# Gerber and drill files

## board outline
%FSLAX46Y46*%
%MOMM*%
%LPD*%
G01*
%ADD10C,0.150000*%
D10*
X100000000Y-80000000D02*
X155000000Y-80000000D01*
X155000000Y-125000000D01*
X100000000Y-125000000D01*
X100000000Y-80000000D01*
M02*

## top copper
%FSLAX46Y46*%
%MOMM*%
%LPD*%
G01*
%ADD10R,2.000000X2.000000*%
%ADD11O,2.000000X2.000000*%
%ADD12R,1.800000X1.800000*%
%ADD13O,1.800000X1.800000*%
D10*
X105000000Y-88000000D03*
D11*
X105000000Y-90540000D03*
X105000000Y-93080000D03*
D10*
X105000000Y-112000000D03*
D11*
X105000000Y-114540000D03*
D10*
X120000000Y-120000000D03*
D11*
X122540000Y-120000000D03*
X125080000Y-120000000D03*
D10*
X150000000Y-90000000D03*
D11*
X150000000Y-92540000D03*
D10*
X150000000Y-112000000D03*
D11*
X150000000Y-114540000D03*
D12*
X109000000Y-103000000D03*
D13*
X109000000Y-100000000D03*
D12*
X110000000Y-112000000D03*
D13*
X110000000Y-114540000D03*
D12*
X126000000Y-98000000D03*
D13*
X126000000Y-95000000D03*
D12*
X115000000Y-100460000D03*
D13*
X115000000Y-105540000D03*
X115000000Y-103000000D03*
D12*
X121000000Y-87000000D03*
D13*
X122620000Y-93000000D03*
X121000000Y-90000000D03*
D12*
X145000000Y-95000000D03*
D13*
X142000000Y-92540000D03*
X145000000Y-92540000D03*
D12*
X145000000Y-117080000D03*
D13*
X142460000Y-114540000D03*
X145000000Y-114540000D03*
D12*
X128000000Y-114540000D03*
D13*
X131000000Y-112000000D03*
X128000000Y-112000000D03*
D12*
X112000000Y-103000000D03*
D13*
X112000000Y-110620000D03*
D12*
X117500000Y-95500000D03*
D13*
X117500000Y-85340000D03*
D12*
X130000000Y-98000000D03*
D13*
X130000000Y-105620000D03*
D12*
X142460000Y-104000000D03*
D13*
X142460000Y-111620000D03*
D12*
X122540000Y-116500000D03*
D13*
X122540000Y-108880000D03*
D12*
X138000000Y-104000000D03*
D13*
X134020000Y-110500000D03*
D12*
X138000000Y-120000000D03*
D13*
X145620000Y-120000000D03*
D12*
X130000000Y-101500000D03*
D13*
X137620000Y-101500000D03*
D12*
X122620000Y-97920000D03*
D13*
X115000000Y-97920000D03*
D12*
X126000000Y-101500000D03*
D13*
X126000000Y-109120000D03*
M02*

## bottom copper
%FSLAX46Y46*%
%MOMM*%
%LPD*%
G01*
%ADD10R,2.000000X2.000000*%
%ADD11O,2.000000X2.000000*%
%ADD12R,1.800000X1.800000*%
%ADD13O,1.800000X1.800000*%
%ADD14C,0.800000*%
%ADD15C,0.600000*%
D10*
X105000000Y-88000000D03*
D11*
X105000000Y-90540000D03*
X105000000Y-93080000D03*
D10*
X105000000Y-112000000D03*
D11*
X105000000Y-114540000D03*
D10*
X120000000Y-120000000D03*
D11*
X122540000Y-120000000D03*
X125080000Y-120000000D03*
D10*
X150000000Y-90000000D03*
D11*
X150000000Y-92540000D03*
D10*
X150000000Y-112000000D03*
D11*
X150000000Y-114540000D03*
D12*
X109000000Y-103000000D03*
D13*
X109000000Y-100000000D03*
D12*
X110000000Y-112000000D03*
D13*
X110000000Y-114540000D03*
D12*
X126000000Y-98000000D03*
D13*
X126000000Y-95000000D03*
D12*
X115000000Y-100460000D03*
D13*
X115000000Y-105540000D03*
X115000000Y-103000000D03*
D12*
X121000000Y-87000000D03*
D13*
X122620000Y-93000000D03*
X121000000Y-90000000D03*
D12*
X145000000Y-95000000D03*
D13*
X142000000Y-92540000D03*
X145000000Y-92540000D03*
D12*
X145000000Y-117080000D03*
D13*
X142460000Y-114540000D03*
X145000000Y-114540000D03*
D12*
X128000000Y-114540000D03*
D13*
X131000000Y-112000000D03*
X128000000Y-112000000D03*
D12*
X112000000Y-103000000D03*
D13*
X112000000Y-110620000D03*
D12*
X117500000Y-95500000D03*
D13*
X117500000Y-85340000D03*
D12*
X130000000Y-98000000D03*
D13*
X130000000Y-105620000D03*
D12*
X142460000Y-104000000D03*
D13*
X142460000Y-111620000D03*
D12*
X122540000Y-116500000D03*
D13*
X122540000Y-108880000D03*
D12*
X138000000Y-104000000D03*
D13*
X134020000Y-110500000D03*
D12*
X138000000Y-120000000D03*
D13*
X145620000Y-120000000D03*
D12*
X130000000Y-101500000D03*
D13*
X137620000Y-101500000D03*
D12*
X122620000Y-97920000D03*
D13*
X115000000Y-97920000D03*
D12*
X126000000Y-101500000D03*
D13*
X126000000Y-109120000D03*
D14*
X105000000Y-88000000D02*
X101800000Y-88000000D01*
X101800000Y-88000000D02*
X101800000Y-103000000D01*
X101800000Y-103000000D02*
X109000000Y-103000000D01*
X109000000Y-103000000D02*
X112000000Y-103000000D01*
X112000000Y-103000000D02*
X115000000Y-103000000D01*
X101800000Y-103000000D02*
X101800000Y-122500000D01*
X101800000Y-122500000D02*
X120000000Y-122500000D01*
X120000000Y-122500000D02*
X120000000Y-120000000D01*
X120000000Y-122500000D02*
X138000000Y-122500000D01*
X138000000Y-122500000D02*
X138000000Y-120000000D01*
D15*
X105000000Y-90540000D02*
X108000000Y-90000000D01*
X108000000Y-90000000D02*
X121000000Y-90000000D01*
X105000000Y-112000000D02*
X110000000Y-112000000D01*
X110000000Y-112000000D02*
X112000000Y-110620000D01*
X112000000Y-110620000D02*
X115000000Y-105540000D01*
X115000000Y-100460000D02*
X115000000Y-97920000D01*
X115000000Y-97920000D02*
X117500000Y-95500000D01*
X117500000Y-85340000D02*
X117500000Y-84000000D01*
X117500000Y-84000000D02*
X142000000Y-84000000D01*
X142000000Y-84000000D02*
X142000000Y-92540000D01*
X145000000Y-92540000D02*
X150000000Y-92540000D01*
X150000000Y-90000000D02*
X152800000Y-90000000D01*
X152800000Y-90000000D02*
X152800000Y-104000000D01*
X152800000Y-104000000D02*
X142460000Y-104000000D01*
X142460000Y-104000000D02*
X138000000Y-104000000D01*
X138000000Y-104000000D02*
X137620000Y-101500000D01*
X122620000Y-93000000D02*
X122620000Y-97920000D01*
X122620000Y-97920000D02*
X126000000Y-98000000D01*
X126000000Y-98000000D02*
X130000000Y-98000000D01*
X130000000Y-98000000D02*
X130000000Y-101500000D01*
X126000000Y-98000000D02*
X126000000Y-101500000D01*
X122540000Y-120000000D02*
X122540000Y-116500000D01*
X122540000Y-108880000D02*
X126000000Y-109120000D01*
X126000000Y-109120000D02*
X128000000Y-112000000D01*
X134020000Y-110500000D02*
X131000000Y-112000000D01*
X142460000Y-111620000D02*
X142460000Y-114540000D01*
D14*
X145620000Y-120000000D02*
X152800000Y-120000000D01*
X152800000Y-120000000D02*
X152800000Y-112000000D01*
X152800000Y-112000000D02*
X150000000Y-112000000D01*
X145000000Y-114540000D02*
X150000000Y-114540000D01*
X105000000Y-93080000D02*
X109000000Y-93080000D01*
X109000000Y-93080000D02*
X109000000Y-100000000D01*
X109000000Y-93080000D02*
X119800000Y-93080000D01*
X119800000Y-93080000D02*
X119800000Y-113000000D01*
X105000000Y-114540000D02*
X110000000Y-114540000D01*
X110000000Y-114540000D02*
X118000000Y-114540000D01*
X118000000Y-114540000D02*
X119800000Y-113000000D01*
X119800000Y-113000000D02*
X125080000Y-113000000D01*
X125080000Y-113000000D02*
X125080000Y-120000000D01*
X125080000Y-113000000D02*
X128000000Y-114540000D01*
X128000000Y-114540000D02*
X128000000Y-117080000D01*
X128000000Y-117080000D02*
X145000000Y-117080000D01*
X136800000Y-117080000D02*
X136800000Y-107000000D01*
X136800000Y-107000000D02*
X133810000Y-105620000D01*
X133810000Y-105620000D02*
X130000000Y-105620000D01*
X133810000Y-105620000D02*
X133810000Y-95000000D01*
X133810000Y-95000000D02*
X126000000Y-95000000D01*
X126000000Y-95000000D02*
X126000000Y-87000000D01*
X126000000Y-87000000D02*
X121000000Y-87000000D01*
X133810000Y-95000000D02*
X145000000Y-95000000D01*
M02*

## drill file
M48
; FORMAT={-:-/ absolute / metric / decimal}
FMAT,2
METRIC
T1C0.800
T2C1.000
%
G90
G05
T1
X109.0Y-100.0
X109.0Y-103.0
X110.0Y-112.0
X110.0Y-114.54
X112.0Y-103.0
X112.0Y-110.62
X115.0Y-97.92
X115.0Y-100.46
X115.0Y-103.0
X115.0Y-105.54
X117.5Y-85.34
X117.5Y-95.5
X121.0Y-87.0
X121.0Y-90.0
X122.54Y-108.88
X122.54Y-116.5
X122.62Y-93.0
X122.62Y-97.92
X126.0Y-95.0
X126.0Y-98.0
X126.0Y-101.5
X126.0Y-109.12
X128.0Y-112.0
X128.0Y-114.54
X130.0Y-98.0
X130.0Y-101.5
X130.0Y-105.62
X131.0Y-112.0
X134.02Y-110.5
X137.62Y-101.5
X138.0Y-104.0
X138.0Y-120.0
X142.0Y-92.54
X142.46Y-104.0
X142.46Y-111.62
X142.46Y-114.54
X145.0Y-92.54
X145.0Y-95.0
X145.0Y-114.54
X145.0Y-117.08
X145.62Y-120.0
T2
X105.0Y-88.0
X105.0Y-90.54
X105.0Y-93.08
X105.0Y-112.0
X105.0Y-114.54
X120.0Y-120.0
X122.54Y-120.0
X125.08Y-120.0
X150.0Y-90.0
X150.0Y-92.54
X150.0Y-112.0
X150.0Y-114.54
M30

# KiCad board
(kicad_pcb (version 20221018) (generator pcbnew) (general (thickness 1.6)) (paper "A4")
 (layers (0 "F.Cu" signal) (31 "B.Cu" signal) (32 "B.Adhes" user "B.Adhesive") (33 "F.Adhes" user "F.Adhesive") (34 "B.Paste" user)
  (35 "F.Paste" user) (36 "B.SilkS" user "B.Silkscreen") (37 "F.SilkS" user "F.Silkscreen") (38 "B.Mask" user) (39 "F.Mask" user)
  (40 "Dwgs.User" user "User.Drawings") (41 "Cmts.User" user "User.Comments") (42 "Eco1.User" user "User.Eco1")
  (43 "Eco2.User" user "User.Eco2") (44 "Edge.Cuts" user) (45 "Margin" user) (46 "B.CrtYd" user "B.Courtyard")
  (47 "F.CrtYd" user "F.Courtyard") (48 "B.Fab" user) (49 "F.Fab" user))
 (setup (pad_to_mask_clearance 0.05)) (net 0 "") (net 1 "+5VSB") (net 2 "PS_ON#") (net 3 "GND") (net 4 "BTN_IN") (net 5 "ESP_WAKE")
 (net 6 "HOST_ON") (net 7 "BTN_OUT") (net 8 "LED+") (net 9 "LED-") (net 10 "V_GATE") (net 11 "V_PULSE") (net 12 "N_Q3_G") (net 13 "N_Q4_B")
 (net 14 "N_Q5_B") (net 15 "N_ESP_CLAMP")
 (gr_rect (start 100 80) (end 155 125) (layer "Edge.Cuts") (width 0.15) (fill none))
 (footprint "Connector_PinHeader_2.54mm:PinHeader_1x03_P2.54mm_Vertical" (layer "F.Cu") (at 105.00 88.00)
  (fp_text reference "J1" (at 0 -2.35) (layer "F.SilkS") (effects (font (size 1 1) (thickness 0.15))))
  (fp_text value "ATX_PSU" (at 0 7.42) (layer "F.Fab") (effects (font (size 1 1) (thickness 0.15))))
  (pad "1" thru_hole rect (at 0.00 0.00) (size 2.00 2.00) (drill 1.00) (layers "B.Cu" "B.Mask") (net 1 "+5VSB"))
  (pad "2" thru_hole oval (at 0.00 2.54) (size 2.00 2.00) (drill 1.00) (layers "B.Cu" "B.Mask") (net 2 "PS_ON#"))
  (pad "3" thru_hole oval (at 0.00 5.08) (size 2.00 2.00) (drill 1.00) (layers "B.Cu" "B.Mask") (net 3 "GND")))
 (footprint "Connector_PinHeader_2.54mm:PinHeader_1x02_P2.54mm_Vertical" (layer "F.Cu") (at 105.00 112.00)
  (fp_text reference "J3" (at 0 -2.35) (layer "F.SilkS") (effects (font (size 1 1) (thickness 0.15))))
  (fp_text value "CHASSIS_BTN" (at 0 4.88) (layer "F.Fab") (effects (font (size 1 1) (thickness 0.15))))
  (pad "1" thru_hole rect (at 0.00 0.00) (size 2.00 2.00) (drill 1.00) (layers "B.Cu" "B.Mask") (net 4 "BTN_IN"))
  (pad "2" thru_hole oval (at 0.00 2.54) (size 2.00 2.00) (drill 1.00) (layers "B.Cu" "B.Mask") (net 3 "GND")))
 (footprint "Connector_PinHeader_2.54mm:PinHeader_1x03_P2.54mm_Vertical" (layer "F.Cu") (at 120.00 120.00)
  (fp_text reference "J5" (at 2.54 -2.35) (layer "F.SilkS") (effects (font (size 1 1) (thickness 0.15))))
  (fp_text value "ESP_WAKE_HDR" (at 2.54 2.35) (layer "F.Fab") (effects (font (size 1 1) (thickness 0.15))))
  (pad "1" thru_hole rect (at 0.00 0.00) (size 2.00 2.00) (drill 1.00) (layers "B.Cu" "B.Mask") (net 1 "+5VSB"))
  (pad "2" thru_hole oval (at 2.54 0.00) (size 2.00 2.00) (drill 1.00) (layers "B.Cu" "B.Mask") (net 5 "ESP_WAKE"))
  (pad "3" thru_hole oval (at 5.08 0.00) (size 2.00 2.00) (drill 1.00) (layers "B.Cu" "B.Mask") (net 3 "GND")))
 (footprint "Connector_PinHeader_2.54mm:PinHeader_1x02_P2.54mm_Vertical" (layer "F.Cu") (at 150.00 90.00)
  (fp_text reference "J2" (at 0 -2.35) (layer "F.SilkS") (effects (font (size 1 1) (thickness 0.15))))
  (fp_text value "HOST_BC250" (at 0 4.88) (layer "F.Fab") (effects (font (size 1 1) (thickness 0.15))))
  (pad "1" thru_hole rect (at 0.00 0.00) (size 2.00 2.00) (drill 1.00) (layers "B.Cu" "B.Mask") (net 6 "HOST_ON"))
  (pad "2" thru_hole oval (at 0.00 2.54) (size 2.00 2.00) (drill 1.00) (layers "B.Cu" "B.Mask") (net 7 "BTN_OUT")))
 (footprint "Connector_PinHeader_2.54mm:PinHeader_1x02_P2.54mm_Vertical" (layer "F.Cu") (at 150.00 112.00)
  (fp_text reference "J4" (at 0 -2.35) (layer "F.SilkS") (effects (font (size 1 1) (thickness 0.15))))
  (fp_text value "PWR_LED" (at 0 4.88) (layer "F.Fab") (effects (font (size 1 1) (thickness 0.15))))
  (pad "1" thru_hole rect (at 0.00 0.00) (size 2.00 2.00) (drill 1.00) (layers "B.Cu" "B.Mask") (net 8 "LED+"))
  (pad "2" thru_hole oval (at 0.00 2.54) (size 2.00 2.00) (drill 1.00) (layers "B.Cu" "B.Mask") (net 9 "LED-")))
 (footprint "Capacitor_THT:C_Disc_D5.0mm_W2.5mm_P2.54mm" (layer "F.Cu") (at 109.00 103.00)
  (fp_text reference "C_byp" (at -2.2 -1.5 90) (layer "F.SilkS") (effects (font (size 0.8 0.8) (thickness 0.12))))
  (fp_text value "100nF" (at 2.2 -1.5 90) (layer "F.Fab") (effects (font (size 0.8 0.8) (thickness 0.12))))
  (pad "1" thru_hole rect (at 0.00 0.00) (size 1.80 1.80) (drill 0.80) (layers "B.Cu" "B.Mask") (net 1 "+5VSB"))
  (pad "2" thru_hole oval (at 0.00 -3.00) (size 1.80 1.80) (drill 0.80) (layers "B.Cu" "B.Mask") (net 3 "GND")))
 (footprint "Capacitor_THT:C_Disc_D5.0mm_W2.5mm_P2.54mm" (layer "F.Cu") (at 110.00 112.00)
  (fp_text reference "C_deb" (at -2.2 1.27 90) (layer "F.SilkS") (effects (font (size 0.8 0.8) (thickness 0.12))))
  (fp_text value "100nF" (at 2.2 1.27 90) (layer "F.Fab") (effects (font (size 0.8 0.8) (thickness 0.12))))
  (pad "1" thru_hole rect (at 0.00 0.00) (size 1.80 1.80) (drill 0.80) (layers "B.Cu" "B.Mask") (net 4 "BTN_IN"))
  (pad "2" thru_hole oval (at 0.00 2.54) (size 1.80 1.80) (drill 0.80) (layers "B.Cu" "B.Mask") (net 3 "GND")))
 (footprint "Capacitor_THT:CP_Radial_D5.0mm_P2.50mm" (layer "F.Cu") (at 126.00 98.00)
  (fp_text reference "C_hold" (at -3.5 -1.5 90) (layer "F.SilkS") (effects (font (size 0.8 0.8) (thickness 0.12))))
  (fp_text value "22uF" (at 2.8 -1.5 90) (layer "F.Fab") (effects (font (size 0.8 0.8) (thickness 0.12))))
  (pad "1" thru_hole rect (at 0.00 0.00) (size 1.80 1.80) (drill 0.80) (layers "B.Cu" "B.Mask") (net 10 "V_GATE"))
  (pad "2" thru_hole oval (at 0.00 -3.00) (size 1.80 1.80) (drill 0.80) (layers "B.Cu" "B.Mask") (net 3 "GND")))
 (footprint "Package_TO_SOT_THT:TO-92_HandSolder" (layer "F.Cu") (at 115.00 103.00)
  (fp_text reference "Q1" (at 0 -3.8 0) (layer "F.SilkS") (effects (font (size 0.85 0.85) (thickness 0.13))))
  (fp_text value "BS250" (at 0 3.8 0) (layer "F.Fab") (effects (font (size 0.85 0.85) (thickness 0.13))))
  (pad "1" thru_hole rect (at 0.00 -2.54) (size 1.80 1.80) (drill 0.80) (layers "B.Cu" "B.Mask") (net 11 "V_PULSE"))
  (pad "2" thru_hole oval (at 0.00 2.54) (size 1.80 1.80) (drill 0.80) (layers "B.Cu" "B.Mask") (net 4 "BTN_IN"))
  (pad "3" thru_hole oval (at 0.00 0.00) (size 1.80 1.80) (drill 0.80) (layers "B.Cu" "B.Mask") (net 1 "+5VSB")))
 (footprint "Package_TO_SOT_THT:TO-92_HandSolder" (layer "F.Cu") (at 121.00 90.00)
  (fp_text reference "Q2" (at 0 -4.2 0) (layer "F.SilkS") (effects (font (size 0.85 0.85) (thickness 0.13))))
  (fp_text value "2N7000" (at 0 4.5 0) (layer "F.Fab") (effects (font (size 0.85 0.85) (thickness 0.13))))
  (pad "1" thru_hole rect (at 0.00 -3.00) (size 1.80 1.80) (drill 0.80) (layers "B.Cu" "B.Mask") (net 3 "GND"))
  (pad "2" thru_hole oval (at 1.62 3.00) (size 1.80 1.80) (drill 0.80) (layers "B.Cu" "B.Mask") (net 10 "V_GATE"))
  (pad "3" thru_hole oval (at 0.00 0.00) (size 1.80 1.80) (drill 0.80) (layers "B.Cu" "B.Mask") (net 2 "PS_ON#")))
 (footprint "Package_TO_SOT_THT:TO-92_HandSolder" (layer "F.Cu") (at 145.00 92.54)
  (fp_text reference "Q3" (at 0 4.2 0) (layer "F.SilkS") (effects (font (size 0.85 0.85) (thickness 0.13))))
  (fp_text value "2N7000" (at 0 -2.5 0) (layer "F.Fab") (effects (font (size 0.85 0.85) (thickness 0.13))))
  (pad "1" thru_hole rect (at 0.00 2.46) (size 1.80 1.80) (drill 0.80) (layers "B.Cu" "B.Mask") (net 3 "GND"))
  (pad "2" thru_hole oval (at -3.00 0.00) (size 1.80 1.80) (drill 0.80) (layers "B.Cu" "B.Mask") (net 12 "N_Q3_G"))
  (pad "3" thru_hole oval (at 0.00 0.00) (size 1.80 1.80) (drill 0.80) (layers "B.Cu" "B.Mask") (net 7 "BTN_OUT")))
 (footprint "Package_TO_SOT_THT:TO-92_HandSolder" (layer "F.Cu") (at 145.00 114.54)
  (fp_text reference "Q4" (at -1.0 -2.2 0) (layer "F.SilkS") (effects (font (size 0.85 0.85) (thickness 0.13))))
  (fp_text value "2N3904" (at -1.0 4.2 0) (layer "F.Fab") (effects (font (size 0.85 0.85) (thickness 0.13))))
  (pad "1" thru_hole rect (at 0.00 2.54) (size 1.80 1.80) (drill 0.80) (layers "B.Cu" "B.Mask") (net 3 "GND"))
  (pad "2" thru_hole oval (at -2.54 0.00) (size 1.80 1.80) (drill 0.80) (layers "B.Cu" "B.Mask") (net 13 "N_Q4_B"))
  (pad "3" thru_hole oval (at 0.00 0.00) (size 1.80 1.80) (drill 0.80) (layers "B.Cu" "B.Mask") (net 9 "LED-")))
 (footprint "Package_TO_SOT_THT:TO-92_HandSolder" (layer "F.Cu") (at 128.00 112.00)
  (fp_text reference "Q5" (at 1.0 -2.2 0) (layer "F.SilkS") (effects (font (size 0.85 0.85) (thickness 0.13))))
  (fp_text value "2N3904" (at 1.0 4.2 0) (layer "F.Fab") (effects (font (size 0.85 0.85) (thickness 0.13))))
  (pad "1" thru_hole rect (at 0.00 2.54) (size 1.80 1.80) (drill 0.80) (layers "B.Cu" "B.Mask") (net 3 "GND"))
  (pad "2" thru_hole oval (at 3.00 0.00) (size 1.80 1.80) (drill 0.80) (layers "B.Cu" "B.Mask") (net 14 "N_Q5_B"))
  (pad "3" thru_hole oval (at 0.00 0.00) (size 1.80 1.80) (drill 0.80) (layers "B.Cu" "B.Mask") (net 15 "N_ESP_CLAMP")))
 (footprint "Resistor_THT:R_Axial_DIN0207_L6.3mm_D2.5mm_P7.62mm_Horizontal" (layer "F.Cu") (at 112.00 103.00)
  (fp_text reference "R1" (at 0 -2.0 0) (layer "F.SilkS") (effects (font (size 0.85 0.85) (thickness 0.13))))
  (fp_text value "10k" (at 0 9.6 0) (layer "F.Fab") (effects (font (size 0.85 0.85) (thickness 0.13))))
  (pad "1" thru_hole rect (at 0.00 0.00) (size 1.80 1.80) (drill 0.80) (layers "B.Cu" "B.Mask") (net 1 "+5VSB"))
  (pad "2" thru_hole oval (at 0.00 7.62) (size 1.80 1.80) (drill 0.80) (layers "B.Cu" "B.Mask") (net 4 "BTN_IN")))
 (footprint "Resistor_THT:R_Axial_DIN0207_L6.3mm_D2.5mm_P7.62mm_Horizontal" (layer "F.Cu") (at 117.50 95.50)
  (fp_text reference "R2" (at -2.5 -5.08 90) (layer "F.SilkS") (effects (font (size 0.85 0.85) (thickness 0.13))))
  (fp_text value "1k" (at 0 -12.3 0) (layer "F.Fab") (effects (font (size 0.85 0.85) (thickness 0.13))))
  (pad "1" thru_hole rect (at 0.00 0.00) (size 1.80 1.80) (drill 0.80) (layers "B.Cu" "B.Mask") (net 11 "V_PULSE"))
  (pad "2" thru_hole oval (at 0.00 -10.16) (size 1.80 1.80) (drill 0.80) (layers "B.Cu" "B.Mask") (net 12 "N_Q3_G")))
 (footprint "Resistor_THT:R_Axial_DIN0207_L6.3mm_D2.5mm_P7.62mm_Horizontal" (layer "F.Cu") (at 130.00 98.00)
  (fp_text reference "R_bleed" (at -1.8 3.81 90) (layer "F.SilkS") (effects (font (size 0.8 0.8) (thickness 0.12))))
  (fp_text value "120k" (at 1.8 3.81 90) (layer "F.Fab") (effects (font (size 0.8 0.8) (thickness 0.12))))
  (pad "1" thru_hole rect (at 0.00 0.00) (size 1.80 1.80) (drill 0.80) (layers "B.Cu" "B.Mask") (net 10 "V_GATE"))
  (pad "2" thru_hole oval (at 0.00 7.62) (size 1.80 1.80) (drill 0.80) (layers "B.Cu" "B.Mask") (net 3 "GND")))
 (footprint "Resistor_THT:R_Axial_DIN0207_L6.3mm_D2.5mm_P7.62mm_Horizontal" (layer "F.Cu") (at 142.46 104.00)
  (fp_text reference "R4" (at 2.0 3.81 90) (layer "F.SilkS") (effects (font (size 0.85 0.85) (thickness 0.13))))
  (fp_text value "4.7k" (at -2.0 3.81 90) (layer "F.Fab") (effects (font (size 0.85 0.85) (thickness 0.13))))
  (pad "1" thru_hole rect (at 0.00 0.00) (size 1.80 1.80) (drill 0.80) (layers "B.Cu" "B.Mask") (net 6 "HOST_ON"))
  (pad "2" thru_hole oval (at 0.00 7.62) (size 1.80 1.80) (drill 0.80) (layers "B.Cu" "B.Mask") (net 13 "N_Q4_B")))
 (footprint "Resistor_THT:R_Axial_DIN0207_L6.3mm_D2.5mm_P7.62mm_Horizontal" (layer "F.Cu") (at 122.54 116.50)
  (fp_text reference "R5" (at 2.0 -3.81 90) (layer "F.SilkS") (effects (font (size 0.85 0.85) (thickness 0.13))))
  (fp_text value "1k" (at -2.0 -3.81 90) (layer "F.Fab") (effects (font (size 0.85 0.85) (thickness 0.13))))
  (pad "1" thru_hole rect (at 0.00 0.00) (size 1.80 1.80) (drill 0.80) (layers "B.Cu" "B.Mask") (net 5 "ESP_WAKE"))
  (pad "2" thru_hole oval (at 0.00 -7.62) (size 1.80 1.80) (drill 0.80) (layers "B.Cu" "B.Mask") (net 15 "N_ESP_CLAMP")))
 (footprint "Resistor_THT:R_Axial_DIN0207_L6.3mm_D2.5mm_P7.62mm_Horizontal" (layer "F.Cu") (at 138.00 104.00)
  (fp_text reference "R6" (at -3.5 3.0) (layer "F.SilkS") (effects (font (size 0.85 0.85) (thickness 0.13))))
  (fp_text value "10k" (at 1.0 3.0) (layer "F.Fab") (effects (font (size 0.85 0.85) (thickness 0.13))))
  (pad "1" thru_hole rect (at 0.00 0.00) (size 1.80 1.80) (drill 0.80) (layers "B.Cu" "B.Mask") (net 6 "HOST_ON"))
  (pad "2" thru_hole oval (at -3.98 6.50) (size 1.80 1.80) (drill 0.80) (layers "B.Cu" "B.Mask") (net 14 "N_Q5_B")))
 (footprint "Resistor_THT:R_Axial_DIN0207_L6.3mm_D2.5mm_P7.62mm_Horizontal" (layer "F.Cu") (at 138.00 120.00)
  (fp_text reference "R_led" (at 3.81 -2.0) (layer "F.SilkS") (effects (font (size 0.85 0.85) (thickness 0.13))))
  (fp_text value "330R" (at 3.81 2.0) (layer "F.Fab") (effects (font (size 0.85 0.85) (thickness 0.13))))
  (pad "1" thru_hole rect (at 0.00 0.00) (size 1.80 1.80) (drill 0.80) (layers "B.Cu" "B.Mask") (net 1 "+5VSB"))
  (pad "2" thru_hole oval (at 7.62 0.00) (size 1.80 1.80) (drill 0.80) (layers "B.Cu" "B.Mask") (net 8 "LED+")))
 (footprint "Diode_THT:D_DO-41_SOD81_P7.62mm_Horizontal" (layer "F.Cu") (at 130.00 101.50)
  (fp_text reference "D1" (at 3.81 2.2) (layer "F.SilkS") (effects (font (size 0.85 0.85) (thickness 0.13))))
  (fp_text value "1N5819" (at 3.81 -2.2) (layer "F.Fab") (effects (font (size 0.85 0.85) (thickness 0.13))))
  (pad "1" thru_hole rect (at 0.00 0.00) (size 1.80 1.80) (drill 0.80) (layers "B.Cu" "B.Mask") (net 10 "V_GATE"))
  (pad "2" thru_hole oval (at 7.62 0.00) (size 1.80 1.80) (drill 0.80) (layers "B.Cu" "B.Mask") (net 6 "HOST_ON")))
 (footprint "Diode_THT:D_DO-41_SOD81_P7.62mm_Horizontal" (layer "F.Cu") (at 122.62 97.92)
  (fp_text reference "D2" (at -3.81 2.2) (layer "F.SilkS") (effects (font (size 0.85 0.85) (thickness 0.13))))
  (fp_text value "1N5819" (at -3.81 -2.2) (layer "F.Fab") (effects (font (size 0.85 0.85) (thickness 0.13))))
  (pad "1" thru_hole rect (at 0.00 0.00) (size 1.80 1.80) (drill 0.80) (layers "B.Cu" "B.Mask") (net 10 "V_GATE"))
  (pad "2" thru_hole oval (at -7.62 0.00) (size 1.80 1.80) (drill 0.80) (layers "B.Cu" "B.Mask") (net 11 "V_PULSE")))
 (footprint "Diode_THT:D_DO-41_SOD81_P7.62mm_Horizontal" (layer "F.Cu") (at 126.00 101.50)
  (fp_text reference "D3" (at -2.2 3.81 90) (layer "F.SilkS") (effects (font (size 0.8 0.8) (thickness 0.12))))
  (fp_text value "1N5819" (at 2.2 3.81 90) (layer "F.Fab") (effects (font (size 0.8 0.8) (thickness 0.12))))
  (pad "1" thru_hole rect (at 0.00 0.00) (size 1.80 1.80) (drill 0.80) (layers "B.Cu" "B.Mask") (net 10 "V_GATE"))
  (pad "2" thru_hole oval (at 0.00 7.62) (size 1.80 1.80) (drill 0.80) (layers "B.Cu" "B.Mask") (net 15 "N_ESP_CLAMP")))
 (segment (start 105.00 88.00) (end 101.80 88.00) (width 0.80) (layer "B.Cu") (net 1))
 (segment (start 101.80 88.00) (end 101.80 103.00) (width 0.80) (layer "B.Cu") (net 1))
 (segment (start 101.80 103.00) (end 109.00 103.00) (width 0.80) (layer "B.Cu") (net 1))
 (segment (start 109.00 103.00) (end 112.00 103.00) (width 0.80) (layer "B.Cu") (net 1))
 (segment (start 112.00 103.00) (end 115.00 103.00) (width 0.80) (layer "B.Cu") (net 1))
 (segment (start 101.80 103.00) (end 101.80 122.50) (width 0.80) (layer "B.Cu") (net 1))
 (segment (start 101.80 122.50) (end 120.00 122.50) (width 0.80) (layer "B.Cu") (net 1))
 (segment (start 120.00 122.50) (end 120.00 120.00) (width 0.80) (layer "B.Cu") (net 1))
 (segment (start 120.00 122.50) (end 138.00 122.50) (width 0.80) (layer "B.Cu") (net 1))
 (segment (start 138.00 122.50) (end 138.00 120.00) (width 0.80) (layer "B.Cu") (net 1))
 (segment (start 105.00 90.54) (end 108.00 90.00) (width 0.60) (layer "B.Cu") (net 2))
 (segment (start 108.00 90.00) (end 121.00 90.00) (width 0.60) (layer "B.Cu") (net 2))
 (segment (start 105.00 112.00) (end 110.00 112.00) (width 0.60) (layer "B.Cu") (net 4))
 (segment (start 110.00 112.00) (end 112.00 110.62) (width 0.60) (layer "B.Cu") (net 4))
 (segment (start 112.00 110.62) (end 115.00 105.54) (width 0.60) (layer "B.Cu") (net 4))
 (segment (start 115.00 100.46) (end 115.00 97.92) (width 0.60) (layer "B.Cu") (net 11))
 (segment (start 115.00 97.92) (end 117.50 95.50) (width 0.60) (layer "B.Cu") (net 11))
 (segment (start 117.50 85.34) (end 117.50 84.00) (width 0.60) (layer "B.Cu") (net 12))
 (segment (start 117.50 84.00) (end 142.00 84.00) (width 0.60) (layer "B.Cu") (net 12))
 (segment (start 142.00 84.00) (end 142.00 92.54) (width 0.60) (layer "B.Cu") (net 12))
 (segment (start 145.00 92.54) (end 150.00 92.54) (width 0.60) (layer "B.Cu") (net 7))
 (segment (start 150.00 90.00) (end 152.80 90.00) (width 0.60) (layer "B.Cu") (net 6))
 (segment (start 152.80 90.00) (end 152.80 104.00) (width 0.60) (layer "B.Cu") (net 6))
 (segment (start 152.80 104.00) (end 142.46 104.00) (width 0.60) (layer "B.Cu") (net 6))
 (segment (start 142.46 104.00) (end 138.00 104.00) (width 0.60) (layer "B.Cu") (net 6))
 (segment (start 138.00 104.00) (end 137.62 101.50) (width 0.60) (layer "B.Cu") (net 6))
 (segment (start 122.62 93.00) (end 122.62 97.92) (width 0.60) (layer "B.Cu") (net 10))
 (segment (start 122.62 97.92) (end 126.00 98.00) (width 0.60) (layer "B.Cu") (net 10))
 (segment (start 126.00 98.00) (end 130.00 98.00) (width 0.60) (layer "B.Cu") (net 10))
 (segment (start 130.00 98.00) (end 130.00 101.50) (width 0.60) (layer "B.Cu") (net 10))
 (segment (start 126.00 98.00) (end 126.00 101.50) (width 0.60) (layer "B.Cu") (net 10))
 (segment (start 122.54 120.00) (end 122.54 116.50) (width 0.60) (layer "B.Cu") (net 5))
 (segment (start 122.54 108.88) (end 126.00 109.12) (width 0.60) (layer "B.Cu") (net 15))
 (segment (start 126.00 109.12) (end 128.00 112.00) (width 0.60) (layer "B.Cu") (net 15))
 (segment (start 134.02 110.50) (end 131.00 112.00) (width 0.60) (layer "B.Cu") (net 14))
 (segment (start 142.46 111.62) (end 142.46 114.54) (width 0.60) (layer "B.Cu") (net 13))
 (segment (start 145.62 120.00) (end 152.80 120.00) (width 0.80) (layer "B.Cu") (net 8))
 (segment (start 152.80 120.00) (end 152.80 112.00) (width 0.80) (layer "B.Cu") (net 8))
 (segment (start 152.80 112.00) (end 150.00 112.00) (width 0.80) (layer "B.Cu") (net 8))
 (segment (start 145.00 114.54) (end 150.00 114.54) (width 0.80) (layer "B.Cu") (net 9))
 (segment (start 105.00 93.08) (end 109.00 93.08) (width 0.80) (layer "B.Cu") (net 3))
 (segment (start 109.00 93.08) (end 109.00 100.00) (width 0.80) (layer "B.Cu") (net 3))
 (segment (start 109.00 93.08) (end 119.80 93.08) (width 0.80) (layer "B.Cu") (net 3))
 (segment (start 119.80 93.08) (end 119.80 113.00) (width 0.80) (layer "B.Cu") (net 3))
 (segment (start 105.00 114.54) (end 110.00 114.54) (width 0.80) (layer "B.Cu") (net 3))
 (segment (start 110.00 114.54) (end 118.00 114.54) (width 0.80) (layer "B.Cu") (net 3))
 (segment (start 118.00 114.54) (end 119.80 113.00) (width 0.80) (layer "B.Cu") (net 3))
 (segment (start 119.80 113.00) (end 125.08 113.00) (width 0.80) (layer "B.Cu") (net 3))
 (segment (start 125.08 113.00) (end 125.08 120.00) (width 0.80) (layer "B.Cu") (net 3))
 (segment (start 125.08 113.00) (end 128.00 114.54) (width 0.80) (layer "B.Cu") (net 3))
 (segment (start 128.00 114.54) (end 128.00 117.08) (width 0.80) (layer "B.Cu") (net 3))
 (segment (start 128.00 117.08) (end 145.00 117.08) (width 0.80) (layer "B.Cu") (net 3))
 (segment (start 136.80 117.08) (end 136.80 107.00) (width 0.80) (layer "B.Cu") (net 3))
 (segment (start 136.80 107.00) (end 133.81 105.62) (width 0.80) (layer "B.Cu") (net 3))
 (segment (start 133.81 105.62) (end 130.00 105.62) (width 0.80) (layer "B.Cu") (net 3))
 (segment (start 133.81 105.62) (end 133.81 95.00) (width 0.80) (layer "B.Cu") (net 3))
 (segment (start 133.81 95.00) (end 126.00 95.00) (width 0.80) (layer "B.Cu") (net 3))
 (segment (start 126.00 95.00) (end 126.00 87.00) (width 0.80) (layer "B.Cu") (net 3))
 (segment (start 126.00 87.00) (end 121.00 87.00) (width 0.80) (layer "B.Cu") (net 3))
 (segment (start 133.81 95.00) (end 145.00 95.00) (width 0.80) (layer "B.Cu") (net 3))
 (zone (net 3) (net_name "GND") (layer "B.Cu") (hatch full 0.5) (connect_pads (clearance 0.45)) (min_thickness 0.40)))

